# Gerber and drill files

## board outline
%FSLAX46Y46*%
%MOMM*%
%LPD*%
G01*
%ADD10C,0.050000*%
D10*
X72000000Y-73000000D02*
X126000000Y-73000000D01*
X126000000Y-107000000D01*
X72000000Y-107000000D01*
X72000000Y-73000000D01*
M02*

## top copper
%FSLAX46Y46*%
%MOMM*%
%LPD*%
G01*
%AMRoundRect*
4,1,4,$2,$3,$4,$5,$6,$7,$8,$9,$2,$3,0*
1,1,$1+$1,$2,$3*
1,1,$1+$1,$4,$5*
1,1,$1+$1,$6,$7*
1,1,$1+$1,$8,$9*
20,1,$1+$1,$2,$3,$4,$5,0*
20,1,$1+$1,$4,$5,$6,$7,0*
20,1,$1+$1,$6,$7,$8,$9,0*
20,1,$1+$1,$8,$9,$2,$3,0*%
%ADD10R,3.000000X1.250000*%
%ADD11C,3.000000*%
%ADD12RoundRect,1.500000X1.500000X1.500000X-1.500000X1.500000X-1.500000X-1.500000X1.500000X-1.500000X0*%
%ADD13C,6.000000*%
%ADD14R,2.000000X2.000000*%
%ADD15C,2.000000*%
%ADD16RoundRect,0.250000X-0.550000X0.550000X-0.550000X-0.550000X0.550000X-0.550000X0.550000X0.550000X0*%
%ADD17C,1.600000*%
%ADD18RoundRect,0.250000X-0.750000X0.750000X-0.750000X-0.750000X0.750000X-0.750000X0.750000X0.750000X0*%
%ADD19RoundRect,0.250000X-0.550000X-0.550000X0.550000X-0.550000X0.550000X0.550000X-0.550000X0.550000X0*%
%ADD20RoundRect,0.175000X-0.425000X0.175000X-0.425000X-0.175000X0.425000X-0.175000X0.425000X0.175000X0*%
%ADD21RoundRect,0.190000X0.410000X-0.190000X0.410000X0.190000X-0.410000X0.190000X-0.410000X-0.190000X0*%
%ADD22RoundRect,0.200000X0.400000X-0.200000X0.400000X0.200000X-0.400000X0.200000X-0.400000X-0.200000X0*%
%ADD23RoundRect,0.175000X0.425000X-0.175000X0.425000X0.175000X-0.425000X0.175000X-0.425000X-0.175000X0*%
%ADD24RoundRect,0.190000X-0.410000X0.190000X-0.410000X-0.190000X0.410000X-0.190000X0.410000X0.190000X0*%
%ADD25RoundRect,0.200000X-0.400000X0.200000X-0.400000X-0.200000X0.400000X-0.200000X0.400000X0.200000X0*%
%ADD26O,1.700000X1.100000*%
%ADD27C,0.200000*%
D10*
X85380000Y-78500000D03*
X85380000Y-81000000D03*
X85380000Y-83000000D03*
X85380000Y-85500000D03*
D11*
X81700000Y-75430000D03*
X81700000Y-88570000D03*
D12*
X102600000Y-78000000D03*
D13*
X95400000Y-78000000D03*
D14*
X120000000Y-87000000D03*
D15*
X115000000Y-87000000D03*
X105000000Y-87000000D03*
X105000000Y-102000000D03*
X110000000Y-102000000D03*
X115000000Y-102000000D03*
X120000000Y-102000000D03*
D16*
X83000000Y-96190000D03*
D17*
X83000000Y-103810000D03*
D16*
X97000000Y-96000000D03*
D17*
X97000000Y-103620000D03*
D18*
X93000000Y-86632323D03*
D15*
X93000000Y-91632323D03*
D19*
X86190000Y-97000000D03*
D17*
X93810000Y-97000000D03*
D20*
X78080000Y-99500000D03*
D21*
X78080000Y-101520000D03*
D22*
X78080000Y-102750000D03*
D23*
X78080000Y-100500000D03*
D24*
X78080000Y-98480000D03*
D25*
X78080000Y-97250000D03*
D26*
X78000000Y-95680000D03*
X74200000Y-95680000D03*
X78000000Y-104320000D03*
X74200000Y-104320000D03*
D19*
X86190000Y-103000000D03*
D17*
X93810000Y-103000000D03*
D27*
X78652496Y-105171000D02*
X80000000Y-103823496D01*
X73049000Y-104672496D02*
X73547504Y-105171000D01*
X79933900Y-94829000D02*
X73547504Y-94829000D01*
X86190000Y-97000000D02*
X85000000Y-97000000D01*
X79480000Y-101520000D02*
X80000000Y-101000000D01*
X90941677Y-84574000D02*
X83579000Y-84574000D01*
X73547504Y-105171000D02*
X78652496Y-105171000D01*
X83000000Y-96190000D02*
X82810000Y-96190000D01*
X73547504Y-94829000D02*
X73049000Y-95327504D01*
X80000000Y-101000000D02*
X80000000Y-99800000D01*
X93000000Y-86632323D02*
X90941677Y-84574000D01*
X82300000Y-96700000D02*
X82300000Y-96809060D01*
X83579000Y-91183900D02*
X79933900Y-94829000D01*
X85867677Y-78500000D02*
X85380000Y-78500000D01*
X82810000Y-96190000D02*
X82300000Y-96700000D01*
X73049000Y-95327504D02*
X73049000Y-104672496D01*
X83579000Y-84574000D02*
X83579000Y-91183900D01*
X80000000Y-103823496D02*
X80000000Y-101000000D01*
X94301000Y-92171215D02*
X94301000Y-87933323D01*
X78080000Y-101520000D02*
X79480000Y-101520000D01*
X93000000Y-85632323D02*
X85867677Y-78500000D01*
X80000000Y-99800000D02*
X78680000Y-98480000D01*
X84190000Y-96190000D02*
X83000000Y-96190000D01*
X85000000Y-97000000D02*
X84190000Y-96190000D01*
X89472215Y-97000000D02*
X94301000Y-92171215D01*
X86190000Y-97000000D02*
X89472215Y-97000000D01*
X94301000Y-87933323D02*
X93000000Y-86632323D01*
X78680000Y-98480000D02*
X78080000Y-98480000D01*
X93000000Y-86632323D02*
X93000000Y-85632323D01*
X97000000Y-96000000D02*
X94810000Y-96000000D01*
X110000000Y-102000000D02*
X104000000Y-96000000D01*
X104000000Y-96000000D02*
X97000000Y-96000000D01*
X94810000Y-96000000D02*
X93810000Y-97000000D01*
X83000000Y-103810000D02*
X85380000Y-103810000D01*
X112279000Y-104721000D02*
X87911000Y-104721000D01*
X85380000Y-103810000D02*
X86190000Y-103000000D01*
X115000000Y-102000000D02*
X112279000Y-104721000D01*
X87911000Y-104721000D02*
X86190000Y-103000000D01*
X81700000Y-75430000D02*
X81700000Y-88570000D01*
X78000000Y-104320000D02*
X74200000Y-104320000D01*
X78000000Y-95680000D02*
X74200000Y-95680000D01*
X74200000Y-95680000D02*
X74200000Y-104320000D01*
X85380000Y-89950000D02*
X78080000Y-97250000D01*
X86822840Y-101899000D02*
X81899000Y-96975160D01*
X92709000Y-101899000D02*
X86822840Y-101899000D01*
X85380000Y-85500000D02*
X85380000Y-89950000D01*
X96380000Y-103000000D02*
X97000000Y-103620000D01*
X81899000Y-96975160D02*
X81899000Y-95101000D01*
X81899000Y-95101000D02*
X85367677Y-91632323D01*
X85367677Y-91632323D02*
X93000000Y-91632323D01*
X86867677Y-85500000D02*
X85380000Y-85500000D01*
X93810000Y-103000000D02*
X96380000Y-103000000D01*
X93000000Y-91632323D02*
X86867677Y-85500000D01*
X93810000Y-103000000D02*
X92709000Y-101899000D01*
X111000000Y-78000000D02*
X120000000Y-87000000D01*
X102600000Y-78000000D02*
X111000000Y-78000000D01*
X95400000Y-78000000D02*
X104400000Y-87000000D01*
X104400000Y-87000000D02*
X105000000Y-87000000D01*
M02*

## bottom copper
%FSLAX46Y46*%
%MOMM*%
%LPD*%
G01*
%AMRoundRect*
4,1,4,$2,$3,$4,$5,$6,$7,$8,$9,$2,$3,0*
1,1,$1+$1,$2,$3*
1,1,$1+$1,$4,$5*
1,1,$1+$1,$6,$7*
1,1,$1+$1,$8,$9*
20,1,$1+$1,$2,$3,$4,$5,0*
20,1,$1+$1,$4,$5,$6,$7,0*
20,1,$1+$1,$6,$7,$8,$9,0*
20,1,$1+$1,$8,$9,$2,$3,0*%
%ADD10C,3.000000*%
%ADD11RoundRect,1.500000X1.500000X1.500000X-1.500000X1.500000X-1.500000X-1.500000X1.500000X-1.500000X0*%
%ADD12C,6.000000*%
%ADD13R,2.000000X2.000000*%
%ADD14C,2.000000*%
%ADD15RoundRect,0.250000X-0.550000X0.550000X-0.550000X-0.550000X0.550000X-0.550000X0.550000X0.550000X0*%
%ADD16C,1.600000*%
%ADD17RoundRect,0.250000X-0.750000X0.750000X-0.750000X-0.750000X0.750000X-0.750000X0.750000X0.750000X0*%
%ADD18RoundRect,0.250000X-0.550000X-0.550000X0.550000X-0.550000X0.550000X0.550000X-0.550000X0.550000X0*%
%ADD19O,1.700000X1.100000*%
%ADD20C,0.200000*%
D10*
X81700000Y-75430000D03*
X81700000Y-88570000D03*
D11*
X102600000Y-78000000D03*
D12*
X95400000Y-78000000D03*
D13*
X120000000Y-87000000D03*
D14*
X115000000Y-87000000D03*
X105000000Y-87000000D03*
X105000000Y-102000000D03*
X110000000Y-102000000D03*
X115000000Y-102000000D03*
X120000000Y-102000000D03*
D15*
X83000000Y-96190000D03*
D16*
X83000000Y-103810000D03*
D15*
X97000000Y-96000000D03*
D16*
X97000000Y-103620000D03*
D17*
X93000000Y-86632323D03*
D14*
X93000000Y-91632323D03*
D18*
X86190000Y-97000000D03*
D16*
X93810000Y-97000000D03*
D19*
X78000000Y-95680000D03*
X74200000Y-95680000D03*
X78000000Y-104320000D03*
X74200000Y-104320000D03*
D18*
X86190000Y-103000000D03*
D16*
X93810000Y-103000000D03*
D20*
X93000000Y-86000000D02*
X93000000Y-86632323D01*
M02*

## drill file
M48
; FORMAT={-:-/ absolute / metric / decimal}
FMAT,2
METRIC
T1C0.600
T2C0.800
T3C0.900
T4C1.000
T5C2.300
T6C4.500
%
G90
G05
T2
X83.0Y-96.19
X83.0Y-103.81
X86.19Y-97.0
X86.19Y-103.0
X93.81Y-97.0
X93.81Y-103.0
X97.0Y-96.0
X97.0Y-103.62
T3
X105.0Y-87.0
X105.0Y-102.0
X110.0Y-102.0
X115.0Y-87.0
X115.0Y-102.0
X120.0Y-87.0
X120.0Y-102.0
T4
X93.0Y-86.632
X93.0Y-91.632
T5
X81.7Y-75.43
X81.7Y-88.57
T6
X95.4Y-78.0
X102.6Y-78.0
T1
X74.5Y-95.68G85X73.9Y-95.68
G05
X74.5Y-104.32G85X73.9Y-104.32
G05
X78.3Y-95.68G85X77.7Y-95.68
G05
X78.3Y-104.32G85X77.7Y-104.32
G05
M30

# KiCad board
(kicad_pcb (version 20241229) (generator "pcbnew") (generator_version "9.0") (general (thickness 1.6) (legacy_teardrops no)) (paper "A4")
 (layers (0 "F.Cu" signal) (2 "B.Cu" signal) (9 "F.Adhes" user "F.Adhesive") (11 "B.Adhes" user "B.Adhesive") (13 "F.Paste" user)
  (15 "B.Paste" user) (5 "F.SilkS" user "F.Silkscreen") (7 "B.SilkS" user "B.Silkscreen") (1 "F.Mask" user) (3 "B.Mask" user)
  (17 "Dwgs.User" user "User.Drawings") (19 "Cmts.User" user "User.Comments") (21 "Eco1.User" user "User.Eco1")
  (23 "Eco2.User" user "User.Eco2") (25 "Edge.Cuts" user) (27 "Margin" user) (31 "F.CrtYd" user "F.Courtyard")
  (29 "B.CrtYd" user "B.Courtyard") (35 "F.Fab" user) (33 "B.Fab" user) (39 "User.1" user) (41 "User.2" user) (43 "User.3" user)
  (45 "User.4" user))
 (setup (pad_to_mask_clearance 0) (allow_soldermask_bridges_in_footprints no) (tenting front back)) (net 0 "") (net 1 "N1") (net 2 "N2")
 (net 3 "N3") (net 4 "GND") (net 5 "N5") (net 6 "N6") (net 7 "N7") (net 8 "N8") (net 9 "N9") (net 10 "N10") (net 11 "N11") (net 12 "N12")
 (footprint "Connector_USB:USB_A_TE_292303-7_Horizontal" (layer "F.Cu") (at 79 82 -90)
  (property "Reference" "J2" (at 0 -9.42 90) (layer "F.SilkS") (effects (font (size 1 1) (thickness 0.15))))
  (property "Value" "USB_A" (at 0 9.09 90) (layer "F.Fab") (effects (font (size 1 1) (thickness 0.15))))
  (pad "1" smd rect (at -3.5 -6.38 270) (size 1.25 3) (layers "F.Cu" "F.Mask" "F.Paste") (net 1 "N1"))
  (pad "2" smd rect (at -1 -6.38 270) (size 1.25 3) (layers "F.Cu" "F.Mask" "F.Paste") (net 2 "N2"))
  (pad "3" smd rect (at 1 -6.38 270) (size 1.25 3) (layers "F.Cu" "F.Mask" "F.Paste") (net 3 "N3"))
  (pad "4" smd rect (at 3.5 -6.38 270) (size 1.25 3) (layers "F.Cu" "F.Mask" "F.Paste") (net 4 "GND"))
  (pad "5" thru_hole circle (at -6.57 -2.7 270) (size 3 3) (drill 2.3) (layers "*.Cu" "*.Mask") (remove_unused_layers no) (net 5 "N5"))
  (pad "5" thru_hole circle (at 6.57 -2.7 270) (size 3 3) (drill 2.3) (layers "*.Cu" "*.Mask") (remove_unused_layers no) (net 5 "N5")))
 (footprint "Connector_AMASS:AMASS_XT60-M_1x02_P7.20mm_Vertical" (layer "F.Cu") (at 102.6 78 180)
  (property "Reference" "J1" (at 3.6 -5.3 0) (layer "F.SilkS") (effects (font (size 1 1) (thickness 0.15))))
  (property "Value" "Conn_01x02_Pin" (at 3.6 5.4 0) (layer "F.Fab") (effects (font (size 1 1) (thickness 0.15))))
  (pad "1" thru_hole roundrect (at 0 0 180) (size 6 6) (drill 4.5) (layers "*.Cu" "*.Mask") (remove_unused_layers no)
   (roundrect_rratio 0.25) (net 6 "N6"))
  (pad "2" thru_hole circle (at 7.2 0 180) (size 6 6) (drill 4.5) (layers "*.Cu" "*.Mask") (remove_unused_layers no) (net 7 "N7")))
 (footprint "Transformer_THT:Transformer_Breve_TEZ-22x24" (layer "F.Cu") (at 120 87 180)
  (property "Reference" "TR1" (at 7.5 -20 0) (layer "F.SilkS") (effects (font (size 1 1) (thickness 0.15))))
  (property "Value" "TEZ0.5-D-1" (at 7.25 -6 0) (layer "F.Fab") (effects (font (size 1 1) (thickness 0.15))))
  (pad "1" thru_hole rect (at 0 0 180) (size 2 2) (drill 0.9) (layers "*.Cu" "*.Mask") (remove_unused_layers no) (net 6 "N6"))
  (pad "2" thru_hole circle (at 5 0 180) (size 2 2) (drill 0.9) (layers "*.Cu" "*.Mask") (remove_unused_layers no))
  (pad "4" thru_hole circle (at 15 0 180) (size 2 2) (drill 0.9) (layers "*.Cu" "*.Mask") (remove_unused_layers no) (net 7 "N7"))
  (pad "5" thru_hole circle (at 15 -15 180) (size 2 2) (drill 0.9) (layers "*.Cu" "*.Mask") (remove_unused_layers no))
  (pad "6" thru_hole circle (at 10 -15 180) (size 2 2) (drill 0.9) (layers "*.Cu" "*.Mask") (remove_unused_layers no) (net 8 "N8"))
  (pad "7" thru_hole circle (at 5 -15 180) (size 2 2) (drill 0.9) (layers "*.Cu" "*.Mask") (remove_unused_layers no) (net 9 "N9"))
  (pad "8" thru_hole circle (at 0 -15 180) (size 2 2) (drill 0.9) (layers "*.Cu" "*.Mask") (remove_unused_layers no)))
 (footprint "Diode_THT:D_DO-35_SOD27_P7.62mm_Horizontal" (layer "F.Cu") (at 83 96.19 -90)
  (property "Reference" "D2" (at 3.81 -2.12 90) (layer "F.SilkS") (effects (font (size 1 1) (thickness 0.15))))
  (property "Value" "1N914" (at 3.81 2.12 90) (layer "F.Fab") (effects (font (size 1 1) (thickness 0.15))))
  (pad "1" thru_hole roundrect (at 0 0 270) (size 1.6 1.6) (drill 0.8) (layers "*.Cu" "*.Mask") (remove_unused_layers no)
   (roundrect_rratio 0.15625) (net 1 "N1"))
  (pad "2" thru_hole circle (at 7.62 0 270) (size 1.6 1.6) (drill 0.8) (layers "*.Cu" "*.Mask") (remove_unused_layers no) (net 9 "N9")))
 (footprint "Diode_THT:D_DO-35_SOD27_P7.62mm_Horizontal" (layer "F.Cu") (at 97 96 -90)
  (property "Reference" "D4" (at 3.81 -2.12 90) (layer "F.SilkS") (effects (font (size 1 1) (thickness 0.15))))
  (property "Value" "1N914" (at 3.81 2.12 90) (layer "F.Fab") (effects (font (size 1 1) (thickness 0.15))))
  (pad "1" thru_hole roundrect (at 0 0 270) (size 1.6 1.6) (drill 0.8) (layers "*.Cu" "*.Mask") (remove_unused_layers no)
   (roundrect_rratio 0.15625) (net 8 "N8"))
  (pad "2" thru_hole circle (at 7.62 0 270) (size 1.6 1.6) (drill 0.8) (layers "*.Cu" "*.Mask") (remove_unused_layers no) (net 4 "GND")))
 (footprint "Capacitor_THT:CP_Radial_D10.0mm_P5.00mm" (layer "F.Cu") (at 93 86.632323 -90)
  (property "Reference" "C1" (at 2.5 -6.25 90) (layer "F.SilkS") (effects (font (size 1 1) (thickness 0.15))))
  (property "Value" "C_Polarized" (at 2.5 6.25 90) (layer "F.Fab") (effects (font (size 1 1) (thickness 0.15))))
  (pad "1" thru_hole roundrect (at 0 0 270) (size 2 2) (drill 1) (layers "*.Cu" "*.Mask") (remove_unused_layers no) (roundrect_rratio 0.125)
   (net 1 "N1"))
  (pad "2" thru_hole circle (at 5 0 270) (size 2 2) (drill 1) (layers "*.Cu" "*.Mask") (remove_unused_layers no) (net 4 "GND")))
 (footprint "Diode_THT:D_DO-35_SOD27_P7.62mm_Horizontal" (layer "F.Cu") (at 86.19 97)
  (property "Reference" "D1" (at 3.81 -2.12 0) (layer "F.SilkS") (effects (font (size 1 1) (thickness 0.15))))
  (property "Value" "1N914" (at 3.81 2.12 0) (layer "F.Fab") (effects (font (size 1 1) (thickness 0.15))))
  (pad "1" thru_hole roundrect (at 0 0) (size 1.6 1.6) (drill 0.8) (layers "*.Cu" "*.Mask") (remove_unused_layers no)
   (roundrect_rratio 0.15625) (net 1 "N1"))
  (pad "2" thru_hole circle (at 7.62 0) (size 1.6 1.6) (drill 0.8) (layers "*.Cu" "*.Mask") (remove_unused_layers no) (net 8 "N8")))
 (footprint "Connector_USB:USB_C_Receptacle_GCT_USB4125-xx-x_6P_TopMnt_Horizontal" (layer "F.Cu") (at 75 100 -90)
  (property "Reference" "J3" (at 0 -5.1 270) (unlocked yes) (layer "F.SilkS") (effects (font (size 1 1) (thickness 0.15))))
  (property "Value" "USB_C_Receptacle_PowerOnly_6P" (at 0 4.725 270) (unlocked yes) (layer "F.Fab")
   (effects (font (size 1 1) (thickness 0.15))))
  (pad "A5" smd roundrect (at -0.5 -3.08 270) (size 0.7 1.2) (layers "F.Cu" "F.Mask" "F.Paste") (roundrect_rratio 0.25) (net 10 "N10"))
  (pad "A9" smd roundrect (at 1.52 -3.08 90) (size 0.76 1.2) (layers "F.Cu" "F.Mask" "F.Paste") (roundrect_rratio 0.25) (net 1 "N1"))
  (pad "A12" smd roundrect (at 2.75 -3.08 90) (size 0.8 1.2) (layers "F.Cu" "F.Mask" "F.Paste") (roundrect_rratio 0.25) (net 4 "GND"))
  (pad "B5" smd roundrect (at 0.5 -3.08 90) (size 0.7 1.2) (layers "F.Cu" "F.Mask" "F.Paste") (roundrect_rratio 0.25) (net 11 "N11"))
  (pad "B9" smd roundrect (at -1.52 -3.08 270) (size 0.76 1.2) (layers "F.Cu" "F.Mask" "F.Paste") (roundrect_rratio 0.25) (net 1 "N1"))
  (pad "B12" smd roundrect (at -2.75 -3.08 270) (size 0.8 1.2) (layers "F.Cu" "F.Mask" "F.Paste") (roundrect_rratio 0.25) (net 4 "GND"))
  (pad "S1" thru_hole oval (at -4.32 -3 270) (size 1.1 1.7) (drill oval 0.6 1.2) (layers "*.Cu" "*.Mask" "F.Paste")
   (remove_unused_layers no) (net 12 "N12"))
  (pad "S1" thru_hole oval (at -4.32 0.8 270) (size 1.1 1.7) (drill oval 0.6 1.2) (layers "*.Cu" "*.Mask" "F.Paste")
   (remove_unused_layers no) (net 12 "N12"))
  (pad "S1" thru_hole oval (at 4.32 -3 270) (size 1.1 1.7) (drill oval 0.6 1.2) (layers "*.Cu" "*.Mask" "F.Paste") (remove_unused_layers no)
   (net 12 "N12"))
  (pad "S1" thru_hole oval (at 4.32 0.8 270) (size 1.1 1.7) (drill oval 0.6 1.2) (layers "*.Cu" "*.Mask" "F.Paste")
   (remove_unused_layers no) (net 12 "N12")))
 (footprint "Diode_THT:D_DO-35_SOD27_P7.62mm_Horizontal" (layer "F.Cu") (at 86.19 103)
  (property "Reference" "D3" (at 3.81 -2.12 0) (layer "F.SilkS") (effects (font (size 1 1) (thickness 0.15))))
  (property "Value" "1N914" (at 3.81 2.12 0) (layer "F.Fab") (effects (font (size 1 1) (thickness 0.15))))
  (pad "1" thru_hole roundrect (at 0 0) (size 1.6 1.6) (drill 0.8) (layers "*.Cu" "*.Mask") (remove_unused_layers no)
   (roundrect_rratio 0.15625) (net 9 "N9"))
  (pad "2" thru_hole circle (at 7.62 0) (size 1.6 1.6) (drill 0.8) (layers "*.Cu" "*.Mask") (remove_unused_layers no) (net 4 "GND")))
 (gr_rect (start 72 73) (end 126 107) (stroke (width 0.05) (type default)) (fill no) (layer "Edge.Cuts"))
 (segment (start 78.652496 105.171) (end 80 103.823496) (width 0.2) (layer "F.Cu") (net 1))
 (segment (start 73.049 104.672496) (end 73.547504 105.171) (width 0.2) (layer "F.Cu") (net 1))
 (segment (start 79.9339 94.829) (end 73.547504 94.829) (width 0.2) (layer "F.Cu") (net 1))
 (segment (start 86.19 97) (end 85 97) (width 0.2) (layer "F.Cu") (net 1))
 (segment (start 79.48 101.52) (end 80 101) (width 0.2) (layer "F.Cu") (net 1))
 (segment (start 90.941677 84.574) (end 83.579 84.574) (width 0.2) (layer "F.Cu") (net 1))
 (segment (start 73.547504 105.171) (end 78.652496 105.171) (width 0.2) (layer "F.Cu") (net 1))
 (segment (start 83 96.19) (end 82.81 96.19) (width 0.2) (layer "F.Cu") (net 1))
 (segment (start 73.547504 94.829) (end 73.049 95.327504) (width 0.2) (layer "F.Cu") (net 1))
 (segment (start 80 101) (end 80 99.8) (width 0.2) (layer "F.Cu") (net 1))
 (segment (start 93 86.632323) (end 90.941677 84.574) (width 0.2) (layer "F.Cu") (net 1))
 (segment (start 82.3 96.7) (end 82.3 96.80906) (width 0.2) (layer "F.Cu") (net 1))
 (segment (start 83.579 91.1839) (end 79.9339 94.829) (width 0.2) (layer "F.Cu") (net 1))
 (segment (start 85.867677 78.5) (end 85.38 78.5) (width 0.2) (layer "F.Cu") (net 1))
 (segment (start 82.81 96.19) (end 82.3 96.7) (width 0.2) (layer "F.Cu") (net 1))
 (segment (start 73.049 95.327504) (end 73.049 104.672496) (width 0.2) (layer "F.Cu") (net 1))
 (segment (start 83.579 84.574) (end 83.579 91.1839) (width 0.2) (layer "F.Cu") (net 1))
 (segment (start 80 103.823496) (end 80 101) (width 0.2) (layer "F.Cu") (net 1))
 (segment (start 94.301 92.171215) (end 94.301 87.933323) (width 0.2) (layer "F.Cu") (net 1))
 (segment (start 78.08 101.52) (end 79.48 101.52) (width 0.2) (layer "F.Cu") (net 1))
 (segment (start 93 85.632323) (end 85.867677 78.5) (width 0.2) (layer "F.Cu") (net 1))
 (segment (start 80 99.8) (end 78.68 98.48) (width 0.2) (layer "F.Cu") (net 1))
 (segment (start 84.19 96.19) (end 83 96.19) (width 0.2) (layer "F.Cu") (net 1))
 (segment (start 85 97) (end 84.19 96.19) (width 0.2) (layer "F.Cu") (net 1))
 (segment (start 89.472215 97) (end 94.301 92.171215) (width 0.2) (layer "F.Cu") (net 1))
 (segment (start 86.19 97) (end 89.472215 97) (width 0.2) (layer "F.Cu") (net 1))
 (segment (start 94.301 87.933323) (end 93 86.632323) (width 0.2) (layer "F.Cu") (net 1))
 (segment (start 78.68 98.48) (end 78.08 98.48) (width 0.2) (layer "F.Cu") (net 1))
 (segment (start 93 86.632323) (end 93 85.632323) (width 0.2) (layer "F.Cu") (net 1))
 (segment (start 93 86) (end 93 86.632323) (width 0.2) (layer "B.Cu") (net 1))
 (segment (start 97 96) (end 94.81 96) (width 0.2) (layer "F.Cu") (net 8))
 (segment (start 110 102) (end 104 96) (width 0.2) (layer "F.Cu") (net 8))
 (segment (start 104 96) (end 97 96) (width 0.2) (layer "F.Cu") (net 8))
 (segment (start 94.81 96) (end 93.81 97) (width 0.2) (layer "F.Cu") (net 8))
 (segment (start 83 103.81) (end 85.38 103.81) (width 0.2) (layer "F.Cu") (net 9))
 (segment (start 112.279 104.721) (end 87.911 104.721) (width 0.2) (layer "F.Cu") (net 9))
 (segment (start 85.38 103.81) (end 86.19 103) (width 0.2) (layer "F.Cu") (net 9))
 (segment (start 115 102) (end 112.279 104.721) (width 0.2) (layer "F.Cu") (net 9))
 (segment (start 87.911 104.721) (end 86.19 103) (width 0.2) (layer "F.Cu") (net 9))
 (segment (start 81.7 75.43) (end 81.7 88.57) (width 0.2) (layer "F.Cu") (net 5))
 (segment (start 78 104.32) (end 74.2 104.32) (width 0.2) (layer "F.Cu") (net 12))
 (segment (start 78 95.68) (end 74.2 95.68) (width 0.2) (layer "F.Cu") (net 12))
 (segment (start 74.2 95.68) (end 74.2 104.32) (width 0.2) (layer "F.Cu") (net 12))
 (segment (start 85.38 89.95) (end 78.08 97.25) (width 0.2) (layer "F.Cu") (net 4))
 (segment (start 86.82284 101.899) (end 81.899 96.97516) (width 0.2) (layer "F.Cu") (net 4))
 (segment (start 92.709 101.899) (end 86.82284 101.899) (width 0.2) (layer "F.Cu") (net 4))
 (segment (start 85.38 85.5) (end 85.38 89.95) (width 0.2) (layer "F.Cu") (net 4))
 (segment (start 96.38 103) (end 97 103.62) (width 0.2) (layer "F.Cu") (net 4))
 (segment (start 81.899 96.97516) (end 81.899 95.101) (width 0.2) (layer "F.Cu") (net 4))
 (segment (start 81.899 95.101) (end 85.367677 91.632323) (width 0.2) (layer "F.Cu") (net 4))
 (segment (start 85.367677 91.632323) (end 93 91.632323) (width 0.2) (layer "F.Cu") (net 4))
 (segment (start 86.867677 85.5) (end 85.38 85.5) (width 0.2) (layer "F.Cu") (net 4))
 (segment (start 93.81 103) (end 96.38 103) (width 0.2) (layer "F.Cu") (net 4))
 (segment (start 93 91.632323) (end 86.867677 85.5) (width 0.2) (layer "F.Cu") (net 4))
 (segment (start 93.81 103) (end 92.709 101.899) (width 0.2) (layer "F.Cu") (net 4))
 (segment (start 111 78) (end 120 87) (width 0.2) (layer "F.Cu") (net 6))
 (segment (start 102.6 78) (end 111 78) (width 0.2) (layer "F.Cu") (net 6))
 (segment (start 95.4 78) (end 104.4 87) (width 0.2) (layer "F.Cu") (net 7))
 (segment (start 104.4 87) (end 105 87) (width 0.2) (layer "F.Cu") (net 7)))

